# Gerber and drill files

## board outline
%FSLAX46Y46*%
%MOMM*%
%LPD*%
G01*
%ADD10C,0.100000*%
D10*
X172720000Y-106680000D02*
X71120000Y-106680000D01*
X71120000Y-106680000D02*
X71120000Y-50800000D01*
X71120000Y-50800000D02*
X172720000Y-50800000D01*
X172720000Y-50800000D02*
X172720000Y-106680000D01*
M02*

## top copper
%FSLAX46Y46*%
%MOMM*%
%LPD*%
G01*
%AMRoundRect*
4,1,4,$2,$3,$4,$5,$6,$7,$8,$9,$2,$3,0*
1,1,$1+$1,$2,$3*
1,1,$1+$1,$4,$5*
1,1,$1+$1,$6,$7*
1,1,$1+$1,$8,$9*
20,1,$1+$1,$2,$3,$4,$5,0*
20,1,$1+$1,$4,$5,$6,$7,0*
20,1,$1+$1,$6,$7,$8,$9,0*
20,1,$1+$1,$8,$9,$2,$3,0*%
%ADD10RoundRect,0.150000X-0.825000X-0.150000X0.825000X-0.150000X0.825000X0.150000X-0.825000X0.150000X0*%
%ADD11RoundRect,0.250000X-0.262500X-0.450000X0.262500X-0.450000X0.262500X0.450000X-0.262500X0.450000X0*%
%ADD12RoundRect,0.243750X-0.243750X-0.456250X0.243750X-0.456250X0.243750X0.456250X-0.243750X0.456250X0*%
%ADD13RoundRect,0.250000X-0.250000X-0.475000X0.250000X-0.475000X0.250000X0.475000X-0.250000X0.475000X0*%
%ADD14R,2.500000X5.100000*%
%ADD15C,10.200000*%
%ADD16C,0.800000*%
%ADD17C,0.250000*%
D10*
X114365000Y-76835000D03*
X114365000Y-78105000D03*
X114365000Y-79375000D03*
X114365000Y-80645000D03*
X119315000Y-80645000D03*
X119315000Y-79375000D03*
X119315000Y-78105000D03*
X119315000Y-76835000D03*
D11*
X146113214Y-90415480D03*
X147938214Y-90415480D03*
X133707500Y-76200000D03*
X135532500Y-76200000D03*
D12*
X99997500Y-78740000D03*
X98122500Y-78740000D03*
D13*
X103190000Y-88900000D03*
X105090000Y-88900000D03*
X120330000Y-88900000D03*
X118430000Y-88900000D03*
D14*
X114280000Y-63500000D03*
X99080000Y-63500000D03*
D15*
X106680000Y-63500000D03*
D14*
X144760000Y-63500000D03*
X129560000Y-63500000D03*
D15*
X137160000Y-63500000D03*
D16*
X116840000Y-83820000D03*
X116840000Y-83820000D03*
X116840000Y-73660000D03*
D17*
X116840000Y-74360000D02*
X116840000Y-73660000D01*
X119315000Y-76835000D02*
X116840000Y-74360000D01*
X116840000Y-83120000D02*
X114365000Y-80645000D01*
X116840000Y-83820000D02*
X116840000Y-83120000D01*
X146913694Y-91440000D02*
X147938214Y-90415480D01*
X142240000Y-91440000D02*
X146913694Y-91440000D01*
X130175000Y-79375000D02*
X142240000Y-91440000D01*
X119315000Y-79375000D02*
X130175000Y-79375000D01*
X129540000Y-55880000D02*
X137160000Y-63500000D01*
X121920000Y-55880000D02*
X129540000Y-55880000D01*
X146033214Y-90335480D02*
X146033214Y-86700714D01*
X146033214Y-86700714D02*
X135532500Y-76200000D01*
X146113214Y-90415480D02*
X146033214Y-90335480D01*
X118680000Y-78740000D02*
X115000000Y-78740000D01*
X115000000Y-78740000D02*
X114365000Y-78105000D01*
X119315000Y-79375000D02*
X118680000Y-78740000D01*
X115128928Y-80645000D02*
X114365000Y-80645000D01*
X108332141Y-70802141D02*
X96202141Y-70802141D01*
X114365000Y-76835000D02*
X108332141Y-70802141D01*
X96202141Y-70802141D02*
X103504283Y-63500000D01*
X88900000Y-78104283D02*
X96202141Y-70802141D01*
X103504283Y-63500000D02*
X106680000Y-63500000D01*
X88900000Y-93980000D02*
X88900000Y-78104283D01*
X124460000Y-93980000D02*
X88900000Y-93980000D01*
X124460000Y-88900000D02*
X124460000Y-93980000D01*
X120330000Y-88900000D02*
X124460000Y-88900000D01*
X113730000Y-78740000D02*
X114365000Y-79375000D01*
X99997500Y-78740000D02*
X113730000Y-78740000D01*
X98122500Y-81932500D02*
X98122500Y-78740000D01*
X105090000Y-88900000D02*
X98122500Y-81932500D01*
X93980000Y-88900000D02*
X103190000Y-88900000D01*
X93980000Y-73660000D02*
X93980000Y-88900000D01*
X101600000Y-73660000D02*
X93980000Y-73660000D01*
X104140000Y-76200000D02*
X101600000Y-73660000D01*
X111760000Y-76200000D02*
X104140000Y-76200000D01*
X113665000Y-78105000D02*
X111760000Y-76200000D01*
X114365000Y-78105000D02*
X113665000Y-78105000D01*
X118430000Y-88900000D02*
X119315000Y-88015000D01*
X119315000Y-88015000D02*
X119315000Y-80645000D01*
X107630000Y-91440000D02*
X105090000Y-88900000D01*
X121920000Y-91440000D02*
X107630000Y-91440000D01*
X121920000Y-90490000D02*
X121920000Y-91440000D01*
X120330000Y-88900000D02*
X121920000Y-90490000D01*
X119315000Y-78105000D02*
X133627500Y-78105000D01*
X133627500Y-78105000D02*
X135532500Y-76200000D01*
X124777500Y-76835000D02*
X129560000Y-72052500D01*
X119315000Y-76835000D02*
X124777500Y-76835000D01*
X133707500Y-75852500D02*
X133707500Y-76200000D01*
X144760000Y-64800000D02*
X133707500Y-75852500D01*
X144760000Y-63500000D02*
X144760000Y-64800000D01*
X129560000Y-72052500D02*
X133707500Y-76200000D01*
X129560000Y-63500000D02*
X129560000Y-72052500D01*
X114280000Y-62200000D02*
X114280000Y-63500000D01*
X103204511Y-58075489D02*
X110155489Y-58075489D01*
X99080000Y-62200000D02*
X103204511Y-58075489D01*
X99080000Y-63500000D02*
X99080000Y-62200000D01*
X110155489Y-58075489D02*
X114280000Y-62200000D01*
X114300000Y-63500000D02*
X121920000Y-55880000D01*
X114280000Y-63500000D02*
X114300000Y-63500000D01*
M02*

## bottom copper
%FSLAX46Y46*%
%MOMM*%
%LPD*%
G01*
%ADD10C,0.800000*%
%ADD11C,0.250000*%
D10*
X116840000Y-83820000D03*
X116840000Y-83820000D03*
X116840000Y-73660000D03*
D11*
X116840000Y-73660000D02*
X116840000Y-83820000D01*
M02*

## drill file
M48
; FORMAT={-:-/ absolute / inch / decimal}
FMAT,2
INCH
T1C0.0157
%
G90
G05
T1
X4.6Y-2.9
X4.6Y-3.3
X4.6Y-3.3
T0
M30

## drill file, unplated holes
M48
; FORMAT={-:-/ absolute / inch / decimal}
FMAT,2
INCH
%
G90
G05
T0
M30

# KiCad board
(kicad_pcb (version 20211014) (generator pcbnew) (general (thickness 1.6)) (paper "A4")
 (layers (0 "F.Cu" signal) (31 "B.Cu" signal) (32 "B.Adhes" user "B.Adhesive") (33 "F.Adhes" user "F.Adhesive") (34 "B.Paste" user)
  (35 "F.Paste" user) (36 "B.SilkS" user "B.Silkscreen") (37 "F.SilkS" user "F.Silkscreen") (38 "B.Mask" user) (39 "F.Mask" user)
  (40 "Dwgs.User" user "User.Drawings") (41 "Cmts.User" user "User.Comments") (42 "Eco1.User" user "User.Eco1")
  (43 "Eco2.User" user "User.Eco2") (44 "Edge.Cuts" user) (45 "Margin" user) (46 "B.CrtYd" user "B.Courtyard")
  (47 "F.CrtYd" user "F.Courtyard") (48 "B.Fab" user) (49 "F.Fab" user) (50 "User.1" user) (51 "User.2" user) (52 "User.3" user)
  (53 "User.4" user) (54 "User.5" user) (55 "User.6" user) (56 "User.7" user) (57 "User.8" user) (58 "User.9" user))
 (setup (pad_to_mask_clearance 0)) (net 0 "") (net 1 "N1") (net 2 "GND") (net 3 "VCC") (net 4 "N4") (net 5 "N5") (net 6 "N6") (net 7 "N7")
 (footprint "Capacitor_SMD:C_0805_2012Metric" (layer "F.Cu") (at 104.14 88.9)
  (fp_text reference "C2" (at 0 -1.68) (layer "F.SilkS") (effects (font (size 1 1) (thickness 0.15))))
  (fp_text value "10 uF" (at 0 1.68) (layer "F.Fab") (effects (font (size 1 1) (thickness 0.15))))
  (pad "1" smd roundrect (at -0.95 0) (size 1 1.45) (layers "F.Cu" "F.Paste" "F.Mask") (roundrect_rratio 0.25) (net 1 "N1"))
  (pad "2" smd roundrect (at 0.95 0) (size 1 1.45) (layers "F.Cu" "F.Paste" "F.Mask") (roundrect_rratio 0.25) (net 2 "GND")))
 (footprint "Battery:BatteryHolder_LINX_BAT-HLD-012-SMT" (layer "F.Cu") (at 137.16 63.5)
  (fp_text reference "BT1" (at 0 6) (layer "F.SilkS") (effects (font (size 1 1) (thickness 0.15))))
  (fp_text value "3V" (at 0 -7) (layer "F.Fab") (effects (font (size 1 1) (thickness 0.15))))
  (pad "1" smd rect (at -7.6 0) (size 2.5 5.1) (layers "F.Cu" "F.Paste" "F.Mask") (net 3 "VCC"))
  (pad "1" smd rect (at 7.6 0) (size 2.5 5.1) (layers "F.Cu" "F.Paste" "F.Mask") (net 3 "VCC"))
  (pad "2" smd circle (at 0 0) (size 10.2 10.2) (layers "F.Cu" "F.Mask") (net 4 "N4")))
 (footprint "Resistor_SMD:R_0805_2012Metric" (layer "F.Cu") (at 134.62 76.2)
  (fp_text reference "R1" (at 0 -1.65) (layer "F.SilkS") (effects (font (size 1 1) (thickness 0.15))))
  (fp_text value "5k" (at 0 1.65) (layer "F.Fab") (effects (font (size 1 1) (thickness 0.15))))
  (pad "1" smd roundrect (at -0.9125 0) (size 1.025 1.4) (layers "F.Cu" "F.Paste" "F.Mask") (roundrect_rratio 0.243902439) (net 3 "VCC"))
  (pad "2" smd roundrect (at 0.9125 0) (size 1.025 1.4) (layers "F.Cu" "F.Paste" "F.Mask") (roundrect_rratio 0.243902439) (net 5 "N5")))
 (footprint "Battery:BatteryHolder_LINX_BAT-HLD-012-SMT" (layer "F.Cu") (at 106.68 63.5)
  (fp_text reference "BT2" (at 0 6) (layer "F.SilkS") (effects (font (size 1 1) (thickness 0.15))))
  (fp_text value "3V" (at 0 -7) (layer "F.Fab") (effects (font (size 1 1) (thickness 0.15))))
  (pad "1" smd rect (at -7.6 0) (size 2.5 5.1) (layers "F.Cu" "F.Paste" "F.Mask") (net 4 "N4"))
  (pad "1" smd rect (at 7.6 0) (size 2.5 5.1) (layers "F.Cu" "F.Paste" "F.Mask") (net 4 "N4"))
  (pad "2" smd circle (at 0 0) (size 10.2 10.2) (layers "F.Cu" "F.Mask") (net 2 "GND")))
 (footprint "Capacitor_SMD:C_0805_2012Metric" (layer "F.Cu") (at 119.38 88.9)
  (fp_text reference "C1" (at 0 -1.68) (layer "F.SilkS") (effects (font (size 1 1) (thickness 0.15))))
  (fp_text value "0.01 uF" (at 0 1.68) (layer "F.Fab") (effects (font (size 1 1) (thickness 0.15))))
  (pad "1" smd roundrect (at -0.95 0) (size 1 1.45) (layers "F.Cu" "F.Paste" "F.Mask") (roundrect_rratio 0.25) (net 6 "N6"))
  (pad "2" smd roundrect (at 0.95 0) (size 1 1.45) (layers "F.Cu" "F.Paste" "F.Mask") (roundrect_rratio 0.25) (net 2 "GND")))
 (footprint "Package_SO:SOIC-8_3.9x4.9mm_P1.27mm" (layer "F.Cu") (at 116.84 78.74)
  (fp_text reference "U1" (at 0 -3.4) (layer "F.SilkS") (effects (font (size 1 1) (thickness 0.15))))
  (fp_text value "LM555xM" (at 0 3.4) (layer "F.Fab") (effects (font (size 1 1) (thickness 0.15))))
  (pad "1" smd roundrect (at -2.475 -1.905) (size 1.95 0.6) (layers "F.Cu" "F.Paste" "F.Mask") (roundrect_rratio 0.25) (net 2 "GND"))
  (pad "2" smd roundrect (at -2.475 -0.635) (size 1.95 0.6) (layers "F.Cu" "F.Paste" "F.Mask") (roundrect_rratio 0.25) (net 1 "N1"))
  (pad "3" smd roundrect (at -2.475 0.635) (size 1.95 0.6) (layers "F.Cu" "F.Paste" "F.Mask") (roundrect_rratio 0.25) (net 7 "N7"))
  (pad "4" smd roundrect (at -2.475 1.905) (size 1.95 0.6) (layers "F.Cu" "F.Paste" "F.Mask") (roundrect_rratio 0.25) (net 3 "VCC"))
  (pad "5" smd roundrect (at 2.475 1.905) (size 1.95 0.6) (layers "F.Cu" "F.Paste" "F.Mask") (roundrect_rratio 0.25) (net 6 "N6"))
  (pad "6" smd roundrect (at 2.475 0.635) (size 1.95 0.6) (layers "F.Cu" "F.Paste" "F.Mask") (roundrect_rratio 0.25) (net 1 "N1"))
  (pad "7" smd roundrect (at 2.475 -0.635) (size 1.95 0.6) (layers "F.Cu" "F.Paste" "F.Mask") (roundrect_rratio 0.25) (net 5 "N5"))
  (pad "8" smd roundrect (at 2.475 -1.905) (size 1.95 0.6) (layers "F.Cu" "F.Paste" "F.Mask") (roundrect_rratio 0.25) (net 3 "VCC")))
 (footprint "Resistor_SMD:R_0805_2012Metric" (layer "F.Cu") (at 147.025714 90.41548)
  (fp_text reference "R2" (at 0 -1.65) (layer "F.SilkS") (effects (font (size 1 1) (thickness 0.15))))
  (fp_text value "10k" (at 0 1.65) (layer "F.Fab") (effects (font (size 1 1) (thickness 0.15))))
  (pad "1" smd roundrect (at -0.9125 0) (size 1.025 1.4) (layers "F.Cu" "F.Paste" "F.Mask") (roundrect_rratio 0.243902439) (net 5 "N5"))
  (pad "2" smd roundrect (at 0.9125 0) (size 1.025 1.4) (layers "F.Cu" "F.Paste" "F.Mask") (roundrect_rratio 0.243902439) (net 1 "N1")))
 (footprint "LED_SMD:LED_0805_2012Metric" (layer "F.Cu") (at 99.06 78.74)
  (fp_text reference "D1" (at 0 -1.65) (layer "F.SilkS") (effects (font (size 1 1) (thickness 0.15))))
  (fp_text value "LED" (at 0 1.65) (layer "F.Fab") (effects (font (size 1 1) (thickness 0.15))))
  (pad "1" smd roundrect (at -0.9375 0) (size 0.975 1.4) (layers "F.Cu" "F.Paste" "F.Mask") (roundrect_rratio 0.25) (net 2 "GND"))
  (pad "2" smd roundrect (at 0.9375 0) (size 0.975 1.4) (layers "F.Cu" "F.Paste" "F.Mask") (roundrect_rratio 0.25) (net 7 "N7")))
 (gr_poly (pts (xy 172.72 106.68) (xy 71.12 106.68) (xy 71.12 50.8) (xy 172.72 50.8)) (layer "Edge.Cuts") (width 0.1) (fill none))
 (segment (start 144.76 63.5) (end 144.76 64.8) (width 0.25) (layer "F.Cu") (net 3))
 (segment (start 129.56 72.0525) (end 133.7075 76.2) (width 0.25) (layer "F.Cu") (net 3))
 (segment (start 133.7075 75.8525) (end 133.7075 76.2) (width 0.25) (layer "F.Cu") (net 3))
 (segment (start 116.84 74.36) (end 116.84 73.66) (width 0.25) (layer "F.Cu") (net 3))
 (segment (start 124.7775 76.835) (end 129.56 72.0525) (width 0.25) (layer "F.Cu") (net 3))
 (segment (start 119.315 76.835) (end 124.7775 76.835) (width 0.25) (layer "F.Cu") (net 3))
 (segment (start 116.84 83.82) (end 116.84 83.12) (width 0.25) (layer "F.Cu") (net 3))
 (segment (start 119.315 76.835) (end 116.84 74.36) (width 0.25) (layer "F.Cu") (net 3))
 (segment (start 116.84 83.12) (end 114.365 80.645) (width 0.25) (layer "F.Cu") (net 3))
 (segment (start 144.76 64.8) (end 133.7075 75.8525) (width 0.25) (layer "F.Cu") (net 3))
 (segment (start 115.128928 80.645) (end 114.365 80.645) (width 0.25) (layer "F.Cu") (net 3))
 (segment (start 129.56 63.5) (end 129.56 72.0525) (width 0.25) (layer "F.Cu") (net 3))
 (via (at 116.84 83.82) (size 0.8) (drill 0.4) (layers "F.Cu" "B.Cu") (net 3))
 (via (at 116.84 83.82) (size 0.8) (drill 0.4) (layers "F.Cu" "B.Cu") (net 3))
 (via (at 116.84 73.66) (size 0.8) (drill 0.4) (layers "F.Cu" "B.Cu") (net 3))
 (segment (start 116.84 73.66) (end 116.84 83.82) (width 0.25) (layer "B.Cu") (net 3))
 (segment (start 114.3 63.5) (end 121.92 55.88) (width 0.25) (layer "F.Cu") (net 4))
 (segment (start 103.204511 58.075489) (end 110.155489 58.075489) (width 0.25) (layer "F.Cu") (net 4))
 (segment (start 99.08 63.5) (end 99.08 62.2) (width 0.25) (layer "F.Cu") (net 4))
 (segment (start 121.92 55.88) (end 129.54 55.88) (width 0.25) (layer "F.Cu") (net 4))
 (segment (start 99.08 62.2) (end 103.204511 58.075489) (width 0.25) (layer "F.Cu") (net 4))
 (segment (start 114.28 62.2) (end 114.28 63.5) (width 0.25) (layer "F.Cu") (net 4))
 (segment (start 110.155489 58.075489) (end 114.28 62.2) (width 0.25) (layer "F.Cu") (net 4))
 (segment (start 114.28 63.5) (end 114.3 63.5) (width 0.25) (layer "F.Cu") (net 4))
 (segment (start 129.54 55.88) (end 137.16 63.5) (width 0.25) (layer "F.Cu") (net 4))
 (segment (start 88.9 93.98) (end 88.9 78.104283) (width 0.25) (layer "F.Cu") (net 2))
 (segment (start 120.33 88.9) (end 121.92 90.49) (width 0.25) (layer "F.Cu") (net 2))
 (segment (start 105.09 88.9) (end 98.1225 81.9325) (width 0.25) (layer "F.Cu") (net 2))
 (segment (start 96.202141 70.802141) (end 103.504283 63.5) (width 0.25) (layer "F.Cu") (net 2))
 (segment (start 103.504283 63.5) (end 106.68 63.5) (width 0.25) (layer "F.Cu") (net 2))
 (segment (start 114.365 76.835) (end 108.332141 70.802141) (width 0.25) (layer "F.Cu") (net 2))
 (segment (start 120.33 88.9) (end 124.46 88.9) (width 0.25) (layer "F.Cu") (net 2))
 (segment (start 121.92 90.49) (end 121.92 91.44) (width 0.25) (layer "F.Cu") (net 2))
 (segment (start 88.9 78.104283) (end 96.202141 70.802141) (width 0.25) (layer "F.Cu") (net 2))
 (segment (start 98.1225 81.9325) (end 98.1225 78.74) (width 0.25) (layer "F.Cu") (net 2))
 (segment (start 124.46 93.98) (end 88.9 93.98) (width 0.25) (layer "F.Cu") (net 2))
 (segment (start 108.332141 70.802141) (end 96.202141 70.802141) (width 0.25) (layer "F.Cu") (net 2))
 (segment (start 107.63 91.44) (end 105.09 88.9) (width 0.25) (layer "F.Cu") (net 2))
 (segment (start 124.46 88.9) (end 124.46 93.98) (width 0.25) (layer "F.Cu") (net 2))
 (segment (start 121.92 91.44) (end 107.63 91.44) (width 0.25) (layer "F.Cu") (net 2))
 (segment (start 118.43 88.9) (end 119.315 88.015) (width 0.25) (layer "F.Cu") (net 6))
 (segment (start 119.315 88.015) (end 119.315 80.645) (width 0.25) (layer "F.Cu") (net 6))
 (segment (start 146.913694 91.44) (end 147.938214 90.41548) (width 0.25) (layer "F.Cu") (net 1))
 (segment (start 111.76 76.2) (end 104.14 76.2) (width 0.25) (layer "F.Cu") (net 1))
 (segment (start 113.665 78.105) (end 111.76 76.2) (width 0.25) (layer "F.Cu") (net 1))
 (segment (start 119.315 79.375) (end 130.175 79.375) (width 0.25) (layer "F.Cu") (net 1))
 (segment (start 130.175 79.375) (end 142.24 91.44) (width 0.25) (layer "F.Cu") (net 1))
 (segment (start 101.6 73.66) (end 93.98 73.66) (width 0.25) (layer "F.Cu") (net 1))
 (segment (start 93.98 73.66) (end 93.98 88.9) (width 0.25) (layer "F.Cu") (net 1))
 (segment (start 119.315 79.375) (end 118.68 78.74) (width 0.25) (layer "F.Cu") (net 1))
 (segment (start 142.24 91.44) (end 146.913694 91.44) (width 0.25) (layer "F.Cu") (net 1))
 (segment (start 93.98 88.9) (end 103.19 88.9) (width 0.25) (layer "F.Cu") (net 1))
 (segment (start 118.68 78.74) (end 115 78.74) (width 0.25) (layer "F.Cu") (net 1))
 (segment (start 114.365 78.105) (end 113.665 78.105) (width 0.25) (layer "F.Cu") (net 1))
 (segment (start 104.14 76.2) (end 101.6 73.66) (width 0.25) (layer "F.Cu") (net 1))
 (segment (start 115 78.74) (end 114.365 78.105) (width 0.25) (layer "F.Cu") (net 1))
 (segment (start 99.9975 78.74) (end 113.73 78.74) (width 0.25) (layer "F.Cu") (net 7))
 (segment (start 113.73 78.74) (end 114.365 79.375) (width 0.25) (layer "F.Cu") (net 7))
 (segment (start 146.033214 90.33548) (end 146.033214 86.700714) (width 0.25) (layer "F.Cu") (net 5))
 (segment (start 146.113214 90.41548) (end 146.033214 90.33548) (width 0.25) (layer "F.Cu") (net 5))
 (segment (start 146.033214 86.700714) (end 135.5325 76.2) (width 0.25) (layer "F.Cu") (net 5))
 (segment (start 133.6275 78.105) (end 135.5325 76.2) (width 0.25) (layer "F.Cu") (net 5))
 (segment (start 119.315 78.105) (end 133.6275 78.105) (width 0.25) (layer "F.Cu") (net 5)))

